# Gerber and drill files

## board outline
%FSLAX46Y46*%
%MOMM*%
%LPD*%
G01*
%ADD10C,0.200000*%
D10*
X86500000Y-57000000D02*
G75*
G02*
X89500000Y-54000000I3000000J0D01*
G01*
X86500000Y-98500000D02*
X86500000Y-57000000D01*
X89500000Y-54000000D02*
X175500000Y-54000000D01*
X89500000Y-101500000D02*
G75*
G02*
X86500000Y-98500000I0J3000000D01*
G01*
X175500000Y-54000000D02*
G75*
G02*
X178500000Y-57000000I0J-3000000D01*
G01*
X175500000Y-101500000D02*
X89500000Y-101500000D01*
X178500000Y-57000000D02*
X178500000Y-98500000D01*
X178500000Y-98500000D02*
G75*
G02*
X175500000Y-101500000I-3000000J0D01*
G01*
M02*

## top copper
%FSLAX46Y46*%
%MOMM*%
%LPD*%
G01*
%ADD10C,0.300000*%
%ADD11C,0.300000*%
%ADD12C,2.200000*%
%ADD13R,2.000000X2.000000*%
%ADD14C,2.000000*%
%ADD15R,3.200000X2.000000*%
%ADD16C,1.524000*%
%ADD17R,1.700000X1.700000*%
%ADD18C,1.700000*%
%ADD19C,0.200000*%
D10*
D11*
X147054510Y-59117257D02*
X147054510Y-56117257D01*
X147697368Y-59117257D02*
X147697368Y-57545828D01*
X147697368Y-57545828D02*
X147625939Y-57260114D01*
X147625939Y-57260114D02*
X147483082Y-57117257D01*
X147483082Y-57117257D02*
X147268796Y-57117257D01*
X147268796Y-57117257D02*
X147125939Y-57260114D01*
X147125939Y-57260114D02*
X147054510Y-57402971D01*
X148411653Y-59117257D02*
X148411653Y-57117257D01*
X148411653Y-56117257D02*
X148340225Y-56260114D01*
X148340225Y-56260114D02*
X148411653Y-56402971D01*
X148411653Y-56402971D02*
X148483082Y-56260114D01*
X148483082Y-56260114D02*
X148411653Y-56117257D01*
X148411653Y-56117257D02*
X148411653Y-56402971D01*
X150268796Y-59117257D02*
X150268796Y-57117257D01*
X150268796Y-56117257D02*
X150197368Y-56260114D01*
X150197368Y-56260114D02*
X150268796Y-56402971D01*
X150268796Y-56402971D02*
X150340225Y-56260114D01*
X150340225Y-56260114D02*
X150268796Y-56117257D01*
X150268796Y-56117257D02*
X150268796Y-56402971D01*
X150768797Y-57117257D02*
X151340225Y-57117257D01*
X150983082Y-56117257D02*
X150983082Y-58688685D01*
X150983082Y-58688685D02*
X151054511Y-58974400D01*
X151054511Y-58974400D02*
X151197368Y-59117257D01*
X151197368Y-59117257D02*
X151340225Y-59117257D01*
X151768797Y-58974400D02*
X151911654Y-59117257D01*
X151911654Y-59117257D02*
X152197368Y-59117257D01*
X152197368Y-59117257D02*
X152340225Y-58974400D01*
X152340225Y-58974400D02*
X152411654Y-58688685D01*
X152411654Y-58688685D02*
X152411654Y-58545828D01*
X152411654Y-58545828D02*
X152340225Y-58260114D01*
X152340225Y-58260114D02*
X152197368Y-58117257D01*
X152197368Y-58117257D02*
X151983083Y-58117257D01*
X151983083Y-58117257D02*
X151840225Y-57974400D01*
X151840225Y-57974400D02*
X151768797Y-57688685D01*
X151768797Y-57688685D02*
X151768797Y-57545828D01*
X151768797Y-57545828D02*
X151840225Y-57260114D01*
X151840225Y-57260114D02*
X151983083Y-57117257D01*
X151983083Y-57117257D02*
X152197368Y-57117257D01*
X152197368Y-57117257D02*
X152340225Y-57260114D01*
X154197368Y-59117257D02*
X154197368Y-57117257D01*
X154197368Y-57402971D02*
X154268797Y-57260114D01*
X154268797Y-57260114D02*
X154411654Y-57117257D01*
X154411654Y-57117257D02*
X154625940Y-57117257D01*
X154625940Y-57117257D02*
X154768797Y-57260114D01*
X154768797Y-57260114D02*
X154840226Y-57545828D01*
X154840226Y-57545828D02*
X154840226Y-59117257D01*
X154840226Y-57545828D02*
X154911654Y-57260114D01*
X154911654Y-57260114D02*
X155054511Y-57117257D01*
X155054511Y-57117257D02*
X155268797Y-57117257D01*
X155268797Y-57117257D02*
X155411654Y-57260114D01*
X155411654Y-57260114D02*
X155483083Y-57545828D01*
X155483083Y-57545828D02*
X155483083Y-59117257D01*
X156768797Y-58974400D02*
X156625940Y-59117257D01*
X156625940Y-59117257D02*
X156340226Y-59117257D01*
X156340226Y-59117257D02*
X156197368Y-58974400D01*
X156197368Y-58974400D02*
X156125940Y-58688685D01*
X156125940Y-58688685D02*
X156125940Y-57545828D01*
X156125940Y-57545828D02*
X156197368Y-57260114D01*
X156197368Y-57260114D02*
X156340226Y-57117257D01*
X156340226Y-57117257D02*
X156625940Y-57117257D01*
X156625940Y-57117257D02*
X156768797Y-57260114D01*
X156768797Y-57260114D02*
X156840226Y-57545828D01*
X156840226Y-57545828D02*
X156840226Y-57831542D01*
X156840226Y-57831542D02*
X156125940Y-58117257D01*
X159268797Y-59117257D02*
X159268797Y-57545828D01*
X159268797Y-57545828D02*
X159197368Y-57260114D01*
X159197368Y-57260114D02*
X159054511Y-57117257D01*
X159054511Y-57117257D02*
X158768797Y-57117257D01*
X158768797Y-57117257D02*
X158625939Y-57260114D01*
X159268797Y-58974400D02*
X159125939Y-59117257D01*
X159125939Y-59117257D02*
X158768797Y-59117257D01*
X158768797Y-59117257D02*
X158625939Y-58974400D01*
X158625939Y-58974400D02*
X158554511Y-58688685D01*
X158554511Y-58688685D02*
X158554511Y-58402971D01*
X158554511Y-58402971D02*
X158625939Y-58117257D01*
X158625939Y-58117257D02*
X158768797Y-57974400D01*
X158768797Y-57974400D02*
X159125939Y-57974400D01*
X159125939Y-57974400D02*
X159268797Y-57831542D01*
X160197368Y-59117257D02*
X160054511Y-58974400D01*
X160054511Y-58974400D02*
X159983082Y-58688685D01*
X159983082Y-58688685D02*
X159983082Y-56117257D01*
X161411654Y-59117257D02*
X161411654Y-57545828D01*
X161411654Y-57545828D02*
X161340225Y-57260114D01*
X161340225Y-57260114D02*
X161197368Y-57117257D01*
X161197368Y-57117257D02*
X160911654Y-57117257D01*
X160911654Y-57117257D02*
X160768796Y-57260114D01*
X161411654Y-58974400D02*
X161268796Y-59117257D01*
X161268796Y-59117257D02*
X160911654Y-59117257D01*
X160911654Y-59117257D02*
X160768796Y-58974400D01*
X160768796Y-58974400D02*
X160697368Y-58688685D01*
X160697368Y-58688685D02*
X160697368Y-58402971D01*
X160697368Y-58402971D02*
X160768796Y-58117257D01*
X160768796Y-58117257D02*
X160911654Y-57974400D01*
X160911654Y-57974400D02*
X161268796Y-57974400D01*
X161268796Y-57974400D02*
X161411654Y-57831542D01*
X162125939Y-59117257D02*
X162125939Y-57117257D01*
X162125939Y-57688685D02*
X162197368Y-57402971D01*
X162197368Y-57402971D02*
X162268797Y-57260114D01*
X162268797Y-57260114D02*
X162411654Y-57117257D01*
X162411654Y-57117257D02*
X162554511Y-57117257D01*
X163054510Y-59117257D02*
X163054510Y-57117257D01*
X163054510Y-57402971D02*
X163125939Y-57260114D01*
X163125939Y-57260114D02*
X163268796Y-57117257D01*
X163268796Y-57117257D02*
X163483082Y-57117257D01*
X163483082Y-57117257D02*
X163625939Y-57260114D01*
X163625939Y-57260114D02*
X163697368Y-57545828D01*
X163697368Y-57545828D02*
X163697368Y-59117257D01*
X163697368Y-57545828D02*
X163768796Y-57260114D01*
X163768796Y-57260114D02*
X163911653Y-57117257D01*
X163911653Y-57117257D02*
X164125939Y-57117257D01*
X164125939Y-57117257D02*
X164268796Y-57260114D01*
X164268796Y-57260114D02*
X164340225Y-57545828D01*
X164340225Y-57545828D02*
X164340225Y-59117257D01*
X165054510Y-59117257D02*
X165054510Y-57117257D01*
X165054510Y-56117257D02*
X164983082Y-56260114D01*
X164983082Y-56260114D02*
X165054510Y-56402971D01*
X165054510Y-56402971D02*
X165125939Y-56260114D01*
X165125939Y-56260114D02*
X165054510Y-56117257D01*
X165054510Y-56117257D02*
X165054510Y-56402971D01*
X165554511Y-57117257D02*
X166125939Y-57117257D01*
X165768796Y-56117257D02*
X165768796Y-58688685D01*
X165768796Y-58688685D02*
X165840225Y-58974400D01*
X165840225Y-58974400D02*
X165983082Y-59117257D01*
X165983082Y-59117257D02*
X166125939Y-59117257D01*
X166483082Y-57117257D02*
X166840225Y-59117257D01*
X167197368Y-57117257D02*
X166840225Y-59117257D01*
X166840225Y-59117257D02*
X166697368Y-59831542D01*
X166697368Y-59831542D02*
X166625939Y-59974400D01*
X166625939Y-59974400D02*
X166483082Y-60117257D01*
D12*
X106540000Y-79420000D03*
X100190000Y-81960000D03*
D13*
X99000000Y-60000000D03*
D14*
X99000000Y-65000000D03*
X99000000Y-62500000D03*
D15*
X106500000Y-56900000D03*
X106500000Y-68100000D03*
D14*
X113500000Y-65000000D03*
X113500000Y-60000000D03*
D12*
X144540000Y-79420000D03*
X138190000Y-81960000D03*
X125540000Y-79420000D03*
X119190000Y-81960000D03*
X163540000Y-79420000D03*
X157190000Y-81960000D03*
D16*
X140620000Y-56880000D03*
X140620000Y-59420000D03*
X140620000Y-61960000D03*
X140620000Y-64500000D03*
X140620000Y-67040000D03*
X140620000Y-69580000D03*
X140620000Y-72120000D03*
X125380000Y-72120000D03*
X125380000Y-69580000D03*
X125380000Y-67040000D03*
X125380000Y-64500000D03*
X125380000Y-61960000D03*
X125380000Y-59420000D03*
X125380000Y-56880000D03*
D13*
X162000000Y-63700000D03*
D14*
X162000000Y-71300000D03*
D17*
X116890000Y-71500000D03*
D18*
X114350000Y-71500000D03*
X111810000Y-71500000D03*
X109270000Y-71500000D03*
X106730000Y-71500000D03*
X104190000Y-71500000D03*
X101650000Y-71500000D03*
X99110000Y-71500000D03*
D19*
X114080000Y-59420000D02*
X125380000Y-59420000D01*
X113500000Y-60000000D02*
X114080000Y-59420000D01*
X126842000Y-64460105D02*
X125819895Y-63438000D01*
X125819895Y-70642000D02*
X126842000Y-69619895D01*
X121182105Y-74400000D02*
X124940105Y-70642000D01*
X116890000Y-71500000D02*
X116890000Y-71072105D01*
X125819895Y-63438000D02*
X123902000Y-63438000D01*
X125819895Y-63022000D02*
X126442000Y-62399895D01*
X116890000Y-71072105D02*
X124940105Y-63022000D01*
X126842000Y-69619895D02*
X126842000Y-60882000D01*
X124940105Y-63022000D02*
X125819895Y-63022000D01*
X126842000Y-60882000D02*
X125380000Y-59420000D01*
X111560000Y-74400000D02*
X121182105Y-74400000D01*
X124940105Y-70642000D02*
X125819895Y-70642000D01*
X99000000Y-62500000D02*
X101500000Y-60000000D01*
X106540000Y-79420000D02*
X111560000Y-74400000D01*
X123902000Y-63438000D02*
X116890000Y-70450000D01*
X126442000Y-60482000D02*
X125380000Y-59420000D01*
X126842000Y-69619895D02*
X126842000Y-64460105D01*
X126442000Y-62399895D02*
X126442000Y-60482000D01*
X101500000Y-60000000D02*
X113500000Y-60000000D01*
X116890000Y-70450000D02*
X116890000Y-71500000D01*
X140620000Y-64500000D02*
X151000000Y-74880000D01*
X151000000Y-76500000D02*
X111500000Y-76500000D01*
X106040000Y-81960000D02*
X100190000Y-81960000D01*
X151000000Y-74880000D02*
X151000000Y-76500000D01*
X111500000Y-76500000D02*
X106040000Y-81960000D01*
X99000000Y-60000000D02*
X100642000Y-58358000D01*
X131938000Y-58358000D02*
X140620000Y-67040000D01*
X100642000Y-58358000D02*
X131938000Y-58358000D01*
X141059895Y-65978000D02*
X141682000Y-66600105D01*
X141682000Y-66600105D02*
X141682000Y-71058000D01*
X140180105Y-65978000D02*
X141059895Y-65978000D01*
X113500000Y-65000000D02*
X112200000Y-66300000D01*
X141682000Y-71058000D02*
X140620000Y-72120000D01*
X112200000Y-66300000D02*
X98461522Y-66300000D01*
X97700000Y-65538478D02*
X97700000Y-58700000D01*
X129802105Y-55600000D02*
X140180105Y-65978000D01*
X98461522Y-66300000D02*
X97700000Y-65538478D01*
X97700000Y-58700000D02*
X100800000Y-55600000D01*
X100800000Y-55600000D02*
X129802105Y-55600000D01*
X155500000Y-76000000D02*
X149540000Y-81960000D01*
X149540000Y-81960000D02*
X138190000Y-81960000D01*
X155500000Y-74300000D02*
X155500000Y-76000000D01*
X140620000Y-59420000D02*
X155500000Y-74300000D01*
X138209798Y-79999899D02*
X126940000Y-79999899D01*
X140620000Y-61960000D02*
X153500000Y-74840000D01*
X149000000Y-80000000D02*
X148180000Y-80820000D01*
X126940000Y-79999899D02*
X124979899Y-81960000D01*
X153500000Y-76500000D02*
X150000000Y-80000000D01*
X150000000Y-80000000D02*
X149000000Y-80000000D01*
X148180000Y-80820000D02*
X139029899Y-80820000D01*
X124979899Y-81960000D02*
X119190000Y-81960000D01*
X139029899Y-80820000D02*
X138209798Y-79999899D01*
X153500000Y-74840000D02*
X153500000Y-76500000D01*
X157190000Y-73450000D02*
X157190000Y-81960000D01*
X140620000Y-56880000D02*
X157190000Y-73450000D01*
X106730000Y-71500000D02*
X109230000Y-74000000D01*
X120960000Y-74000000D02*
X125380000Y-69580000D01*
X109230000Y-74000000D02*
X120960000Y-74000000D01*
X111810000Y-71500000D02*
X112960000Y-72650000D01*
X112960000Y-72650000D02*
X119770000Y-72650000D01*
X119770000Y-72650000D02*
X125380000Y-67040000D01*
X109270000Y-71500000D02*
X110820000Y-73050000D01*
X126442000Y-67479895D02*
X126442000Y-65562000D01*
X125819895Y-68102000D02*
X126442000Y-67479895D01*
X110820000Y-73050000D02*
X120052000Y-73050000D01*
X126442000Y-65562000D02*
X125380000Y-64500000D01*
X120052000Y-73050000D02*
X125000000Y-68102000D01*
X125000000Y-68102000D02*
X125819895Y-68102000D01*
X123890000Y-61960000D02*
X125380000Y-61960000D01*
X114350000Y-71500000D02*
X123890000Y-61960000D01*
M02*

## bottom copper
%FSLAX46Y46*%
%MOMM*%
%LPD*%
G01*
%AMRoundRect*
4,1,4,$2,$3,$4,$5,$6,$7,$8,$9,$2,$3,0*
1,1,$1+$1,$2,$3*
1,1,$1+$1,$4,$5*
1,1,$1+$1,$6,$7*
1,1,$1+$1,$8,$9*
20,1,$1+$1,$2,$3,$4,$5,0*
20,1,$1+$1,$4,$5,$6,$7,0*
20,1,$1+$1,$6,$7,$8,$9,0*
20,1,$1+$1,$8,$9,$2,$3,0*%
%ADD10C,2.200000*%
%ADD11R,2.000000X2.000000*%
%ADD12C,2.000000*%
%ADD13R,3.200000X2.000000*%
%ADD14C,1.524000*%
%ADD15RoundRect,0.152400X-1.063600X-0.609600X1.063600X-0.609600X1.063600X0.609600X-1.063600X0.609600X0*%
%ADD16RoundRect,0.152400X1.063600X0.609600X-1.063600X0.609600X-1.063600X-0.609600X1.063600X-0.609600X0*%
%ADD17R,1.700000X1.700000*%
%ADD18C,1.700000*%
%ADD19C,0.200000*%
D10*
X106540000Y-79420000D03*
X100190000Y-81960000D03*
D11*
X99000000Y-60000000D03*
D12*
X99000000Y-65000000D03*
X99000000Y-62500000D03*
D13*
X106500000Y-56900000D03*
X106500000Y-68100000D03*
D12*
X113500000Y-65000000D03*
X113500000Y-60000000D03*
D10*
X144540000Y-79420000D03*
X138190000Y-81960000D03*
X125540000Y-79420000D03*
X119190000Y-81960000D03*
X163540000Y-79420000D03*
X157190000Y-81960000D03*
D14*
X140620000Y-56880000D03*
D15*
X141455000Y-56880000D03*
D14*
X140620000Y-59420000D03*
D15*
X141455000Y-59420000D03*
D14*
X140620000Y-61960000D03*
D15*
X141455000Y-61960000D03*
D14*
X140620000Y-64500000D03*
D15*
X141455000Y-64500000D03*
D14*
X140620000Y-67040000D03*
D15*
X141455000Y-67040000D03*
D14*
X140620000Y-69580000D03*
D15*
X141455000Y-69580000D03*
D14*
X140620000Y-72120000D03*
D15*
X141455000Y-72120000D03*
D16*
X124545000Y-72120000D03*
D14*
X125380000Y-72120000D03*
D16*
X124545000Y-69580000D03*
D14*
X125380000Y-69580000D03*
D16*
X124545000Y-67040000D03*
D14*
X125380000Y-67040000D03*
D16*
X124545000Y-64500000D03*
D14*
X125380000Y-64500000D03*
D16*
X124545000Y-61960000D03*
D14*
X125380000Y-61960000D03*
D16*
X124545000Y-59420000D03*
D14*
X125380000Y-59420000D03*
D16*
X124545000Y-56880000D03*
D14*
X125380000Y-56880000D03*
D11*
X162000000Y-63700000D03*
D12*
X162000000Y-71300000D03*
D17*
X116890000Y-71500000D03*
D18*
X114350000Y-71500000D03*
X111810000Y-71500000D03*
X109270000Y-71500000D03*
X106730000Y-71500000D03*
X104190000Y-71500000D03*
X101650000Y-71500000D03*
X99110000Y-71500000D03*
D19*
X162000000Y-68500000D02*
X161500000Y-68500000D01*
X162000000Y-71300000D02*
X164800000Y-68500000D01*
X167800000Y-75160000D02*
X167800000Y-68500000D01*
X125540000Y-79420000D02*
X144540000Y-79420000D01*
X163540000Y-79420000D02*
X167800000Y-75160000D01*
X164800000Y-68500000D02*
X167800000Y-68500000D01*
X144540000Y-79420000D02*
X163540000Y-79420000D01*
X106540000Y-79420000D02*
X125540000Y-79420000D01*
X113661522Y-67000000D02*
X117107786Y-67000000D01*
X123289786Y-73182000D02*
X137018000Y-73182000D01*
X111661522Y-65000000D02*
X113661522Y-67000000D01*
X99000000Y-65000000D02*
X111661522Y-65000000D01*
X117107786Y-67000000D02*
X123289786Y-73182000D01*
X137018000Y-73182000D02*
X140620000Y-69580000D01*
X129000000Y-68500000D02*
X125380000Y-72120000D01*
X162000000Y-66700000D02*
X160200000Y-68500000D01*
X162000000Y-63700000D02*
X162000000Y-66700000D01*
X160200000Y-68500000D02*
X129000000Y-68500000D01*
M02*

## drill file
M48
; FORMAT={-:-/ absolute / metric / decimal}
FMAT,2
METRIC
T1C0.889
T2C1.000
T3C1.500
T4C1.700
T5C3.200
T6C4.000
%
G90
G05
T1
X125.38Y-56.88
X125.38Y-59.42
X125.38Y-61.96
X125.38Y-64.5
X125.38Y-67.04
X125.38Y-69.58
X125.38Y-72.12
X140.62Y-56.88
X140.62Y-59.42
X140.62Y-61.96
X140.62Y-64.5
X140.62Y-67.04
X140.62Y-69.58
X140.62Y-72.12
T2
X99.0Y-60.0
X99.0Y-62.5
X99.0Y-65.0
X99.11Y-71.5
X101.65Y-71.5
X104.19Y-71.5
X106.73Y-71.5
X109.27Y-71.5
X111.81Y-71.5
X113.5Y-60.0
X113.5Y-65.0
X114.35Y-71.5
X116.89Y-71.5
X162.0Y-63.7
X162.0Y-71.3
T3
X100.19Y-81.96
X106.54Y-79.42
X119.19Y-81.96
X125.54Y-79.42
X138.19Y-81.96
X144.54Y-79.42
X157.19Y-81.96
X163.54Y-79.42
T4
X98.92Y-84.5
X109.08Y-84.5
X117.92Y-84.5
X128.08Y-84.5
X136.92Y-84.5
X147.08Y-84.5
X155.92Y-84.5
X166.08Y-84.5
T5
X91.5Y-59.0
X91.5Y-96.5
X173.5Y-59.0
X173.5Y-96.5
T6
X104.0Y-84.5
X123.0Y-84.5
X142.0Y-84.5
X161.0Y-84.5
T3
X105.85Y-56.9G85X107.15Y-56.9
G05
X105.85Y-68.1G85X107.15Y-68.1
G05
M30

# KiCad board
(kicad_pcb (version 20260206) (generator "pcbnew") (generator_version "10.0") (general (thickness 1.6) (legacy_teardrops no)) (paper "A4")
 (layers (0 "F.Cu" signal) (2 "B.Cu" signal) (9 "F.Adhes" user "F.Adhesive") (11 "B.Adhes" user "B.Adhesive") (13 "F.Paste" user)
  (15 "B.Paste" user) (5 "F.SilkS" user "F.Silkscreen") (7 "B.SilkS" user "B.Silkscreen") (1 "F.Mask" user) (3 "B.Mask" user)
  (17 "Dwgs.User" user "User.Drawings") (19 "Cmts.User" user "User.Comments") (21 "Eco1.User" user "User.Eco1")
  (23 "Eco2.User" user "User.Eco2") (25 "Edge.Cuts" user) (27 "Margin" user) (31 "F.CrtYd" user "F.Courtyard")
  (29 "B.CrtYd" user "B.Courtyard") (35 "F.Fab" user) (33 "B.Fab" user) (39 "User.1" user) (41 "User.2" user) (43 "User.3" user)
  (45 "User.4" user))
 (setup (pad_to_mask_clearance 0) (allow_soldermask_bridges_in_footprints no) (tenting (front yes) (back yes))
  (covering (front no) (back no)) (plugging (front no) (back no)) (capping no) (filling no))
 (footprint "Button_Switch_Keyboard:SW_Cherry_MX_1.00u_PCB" (layer "F.Cu") (at 106.54 79.42)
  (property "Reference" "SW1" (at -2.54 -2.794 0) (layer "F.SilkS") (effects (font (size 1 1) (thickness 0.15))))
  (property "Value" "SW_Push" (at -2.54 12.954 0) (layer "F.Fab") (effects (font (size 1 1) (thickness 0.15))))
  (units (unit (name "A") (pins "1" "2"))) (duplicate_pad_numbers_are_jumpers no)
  (pad "" np_thru_hole circle (at -7.62 5.08) (size 1.7 1.7) (drill 1.7) (layers "*.Cu" "*.Mask"))
  (pad "" np_thru_hole circle (at -2.54 5.08) (size 4 4) (drill 4) (layers "*.Cu" "*.Mask"))
  (pad "" np_thru_hole circle (at 2.54 5.08) (size 1.7 1.7) (drill 1.7) (layers "*.Cu" "*.Mask"))
  (pad "1" thru_hole circle (at 0 0) (size 2.2 2.2) (drill 1.5) (layers "*.Cu" "*.Mask") (remove_unused_layers no) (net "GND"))
  (pad "2" thru_hole circle (at -6.35 2.54) (size 2.2 2.2) (drill 1.5) (layers "*.Cu" "*.Mask") (remove_unused_layers no)
   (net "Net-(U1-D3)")))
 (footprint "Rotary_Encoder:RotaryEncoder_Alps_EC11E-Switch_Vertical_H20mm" (layer "F.Cu") (at 99 60)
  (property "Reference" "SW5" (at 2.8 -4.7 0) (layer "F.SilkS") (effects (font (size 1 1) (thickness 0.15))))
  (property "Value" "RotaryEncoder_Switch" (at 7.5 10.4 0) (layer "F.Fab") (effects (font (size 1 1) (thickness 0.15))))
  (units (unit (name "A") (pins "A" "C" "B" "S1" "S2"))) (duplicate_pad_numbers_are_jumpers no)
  (pad "A" thru_hole rect (at 0 0) (size 2 2) (drill 1) (layers "*.Cu" "*.Mask") (remove_unused_layers no) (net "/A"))
  (pad "B" thru_hole circle (at 0 5) (size 2 2) (drill 1) (layers "*.Cu" "*.Mask") (remove_unused_layers no) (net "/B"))
  (pad "C" thru_hole circle (at 0 2.5) (size 2 2) (drill 1) (layers "*.Cu" "*.Mask") (remove_unused_layers no) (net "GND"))
  (pad "MP" thru_hole rect (at 7.5 -3.1) (size 3.2 2) (drill oval 2.8 1.5) (layers "*.Cu" "*.Mask") (remove_unused_layers no))
  (pad "MP" thru_hole rect (at 7.5 8.1) (size 3.2 2) (drill oval 2.8 1.5) (layers "*.Cu" "*.Mask") (remove_unused_layers no))
  (pad "S1" thru_hole circle (at 14.5 5) (size 2 2) (drill 1) (layers "*.Cu" "*.Mask") (remove_unused_layers no) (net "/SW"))
  (pad "S2" thru_hole circle (at 14.5 0) (size 2 2) (drill 1) (layers "*.Cu" "*.Mask") (remove_unused_layers no) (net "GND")))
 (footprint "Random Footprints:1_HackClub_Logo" (layer "F.Cu") (at 155.5 68.5)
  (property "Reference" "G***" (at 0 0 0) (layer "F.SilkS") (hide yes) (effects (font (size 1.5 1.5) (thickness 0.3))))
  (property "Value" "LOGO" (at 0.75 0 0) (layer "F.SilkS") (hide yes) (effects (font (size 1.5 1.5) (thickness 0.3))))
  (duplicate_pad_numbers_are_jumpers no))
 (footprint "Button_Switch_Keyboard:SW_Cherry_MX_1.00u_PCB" (layer "F.Cu") (at 144.54 79.42)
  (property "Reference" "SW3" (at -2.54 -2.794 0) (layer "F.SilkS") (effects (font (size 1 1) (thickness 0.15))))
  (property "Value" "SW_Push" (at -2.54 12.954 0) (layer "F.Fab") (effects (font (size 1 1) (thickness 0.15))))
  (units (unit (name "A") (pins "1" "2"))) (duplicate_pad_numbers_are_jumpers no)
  (pad "" np_thru_hole circle (at -7.62 5.08) (size 1.7 1.7) (drill 1.7) (layers "*.Cu" "*.Mask"))
  (pad "" np_thru_hole circle (at -2.54 5.08) (size 4 4) (drill 4) (layers "*.Cu" "*.Mask"))
  (pad "" np_thru_hole circle (at 2.54 5.08) (size 1.7 1.7) (drill 1.7) (layers "*.Cu" "*.Mask"))
  (pad "1" thru_hole circle (at 0 0) (size 2.2 2.2) (drill 1.5) (layers "*.Cu" "*.Mask") (remove_unused_layers no) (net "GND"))
  (pad "2" thru_hole circle (at -6.35 2.54) (size 2.2 2.2) (drill 1.5) (layers "*.Cu" "*.Mask") (remove_unused_layers no)
   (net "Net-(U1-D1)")))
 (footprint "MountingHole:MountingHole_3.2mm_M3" (layer "F.Cu") (at 91.5 96.5 180)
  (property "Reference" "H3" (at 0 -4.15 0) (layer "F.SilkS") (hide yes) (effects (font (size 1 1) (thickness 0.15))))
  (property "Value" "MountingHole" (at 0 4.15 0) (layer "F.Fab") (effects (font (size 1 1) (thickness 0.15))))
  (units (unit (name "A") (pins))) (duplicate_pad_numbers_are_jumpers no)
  (pad "" np_thru_hole circle (at 0 0 180) (size 3.2 3.2) (drill 3.2) (layers "*.Cu" "*.Mask")))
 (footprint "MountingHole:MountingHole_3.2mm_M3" (layer "F.Cu") (at 91.5 59)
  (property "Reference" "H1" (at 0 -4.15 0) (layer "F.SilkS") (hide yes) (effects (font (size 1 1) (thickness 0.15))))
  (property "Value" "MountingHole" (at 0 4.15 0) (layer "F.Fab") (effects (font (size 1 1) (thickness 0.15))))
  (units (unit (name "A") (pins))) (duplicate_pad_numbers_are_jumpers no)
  (pad "" np_thru_hole circle (at 0 0) (size 3.2 3.2) (drill 3.2) (layers "*.Cu" "*.Mask")))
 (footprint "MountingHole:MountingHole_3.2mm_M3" (layer "F.Cu") (at 173.5 59)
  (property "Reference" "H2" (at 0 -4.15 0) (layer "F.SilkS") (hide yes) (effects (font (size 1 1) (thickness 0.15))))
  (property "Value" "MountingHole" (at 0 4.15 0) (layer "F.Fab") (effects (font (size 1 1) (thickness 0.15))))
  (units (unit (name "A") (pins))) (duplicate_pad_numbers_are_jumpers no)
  (pad "" np_thru_hole circle (at 0 0) (size 3.2 3.2) (drill 3.2) (layers "*.Cu" "*.Mask")))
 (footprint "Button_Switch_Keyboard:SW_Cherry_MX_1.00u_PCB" (layer "F.Cu") (at 125.54 79.42)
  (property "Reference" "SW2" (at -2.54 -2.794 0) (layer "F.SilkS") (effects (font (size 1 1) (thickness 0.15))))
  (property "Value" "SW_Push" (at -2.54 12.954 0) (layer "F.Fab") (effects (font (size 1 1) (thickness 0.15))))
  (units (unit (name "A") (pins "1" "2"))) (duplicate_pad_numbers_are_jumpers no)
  (pad "" np_thru_hole circle (at -7.62 5.08) (size 1.7 1.7) (drill 1.7) (layers "*.Cu" "*.Mask"))
  (pad "" np_thru_hole circle (at -2.54 5.08) (size 4 4) (drill 4) (layers "*.Cu" "*.Mask"))
  (pad "" np_thru_hole circle (at 2.54 5.08) (size 1.7 1.7) (drill 1.7) (layers "*.Cu" "*.Mask"))
  (pad "1" thru_hole circle (at 0 0) (size 2.2 2.2) (drill 1.5) (layers "*.Cu" "*.Mask") (remove_unused_layers no) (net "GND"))
  (pad "2" thru_hole circle (at -6.35 2.54) (size 2.2 2.2) (drill 1.5) (layers "*.Cu" "*.Mask") (remove_unused_layers no)
   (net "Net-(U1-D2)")))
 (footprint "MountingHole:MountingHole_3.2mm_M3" (layer "F.Cu") (at 173.5 96.5 180)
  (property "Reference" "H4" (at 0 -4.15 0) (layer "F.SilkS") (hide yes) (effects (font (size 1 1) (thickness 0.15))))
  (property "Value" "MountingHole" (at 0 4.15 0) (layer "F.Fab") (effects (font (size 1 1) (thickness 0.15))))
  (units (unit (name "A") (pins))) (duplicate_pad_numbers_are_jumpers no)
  (pad "" np_thru_hole circle (at 0 0 180) (size 3.2 3.2) (drill 3.2) (layers "*.Cu" "*.Mask")))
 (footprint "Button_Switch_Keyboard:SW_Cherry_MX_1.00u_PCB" (layer "F.Cu") (at 163.54 79.42)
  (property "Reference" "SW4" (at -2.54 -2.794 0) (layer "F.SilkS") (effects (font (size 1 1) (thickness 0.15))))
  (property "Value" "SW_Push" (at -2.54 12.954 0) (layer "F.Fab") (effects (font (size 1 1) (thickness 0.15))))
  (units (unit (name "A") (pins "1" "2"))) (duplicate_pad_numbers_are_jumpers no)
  (pad "" np_thru_hole circle (at -7.62 5.08) (size 1.7 1.7) (drill 1.7) (layers "*.Cu" "*.Mask"))
  (pad "" np_thru_hole circle (at -2.54 5.08) (size 4 4) (drill 4) (layers "*.Cu" "*.Mask"))
  (pad "" np_thru_hole circle (at 2.54 5.08) (size 1.7 1.7) (drill 1.7) (layers "*.Cu" "*.Mask"))
  (pad "1" thru_hole circle (at 0 0) (size 2.2 2.2) (drill 1.5) (layers "*.Cu" "*.Mask") (remove_unused_layers no) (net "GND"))
  (pad "2" thru_hole circle (at -6.35 2.54) (size 2.2 2.2) (drill 1.5) (layers "*.Cu" "*.Mask") (remove_unused_layers no)
   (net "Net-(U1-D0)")))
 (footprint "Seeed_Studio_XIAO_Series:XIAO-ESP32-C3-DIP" (layer "B.Cu") (at 133 64.5 90)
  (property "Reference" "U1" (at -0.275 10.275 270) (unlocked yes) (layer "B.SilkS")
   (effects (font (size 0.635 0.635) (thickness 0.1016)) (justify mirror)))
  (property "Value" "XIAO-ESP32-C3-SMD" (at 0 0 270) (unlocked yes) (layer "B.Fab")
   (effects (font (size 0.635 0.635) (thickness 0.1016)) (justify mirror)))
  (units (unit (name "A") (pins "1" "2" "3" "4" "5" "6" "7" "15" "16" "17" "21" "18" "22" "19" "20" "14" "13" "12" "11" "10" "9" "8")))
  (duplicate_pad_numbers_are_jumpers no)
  (pad "1" thru_hole circle (at 7.62 7.62) (size 1.524 1.524) (drill 0.889) (layers "*.Cu" "*.Mask") (remove_unused_layers no)
   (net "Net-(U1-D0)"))
  (pad "1" smd roundrect (at 7.62 8.455) (size 2.432 1.524) (layers "B.Cu" "B.Mask") (roundrect_rratio 0.1) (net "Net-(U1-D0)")
   (thermal_bridge_angle 45))
  (pad "2" thru_hole circle (at 5.08 7.62) (size 1.524 1.524) (drill 0.889) (layers "*.Cu" "*.Mask") (remove_unused_layers no)
   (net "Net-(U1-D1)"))
  (pad "2" smd roundrect (at 5.08 8.455) (size 2.432 1.524) (layers "B.Cu" "B.Mask") (roundrect_rratio 0.1) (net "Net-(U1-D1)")
   (thermal_bridge_angle 45))
  (pad "3" thru_hole circle (at 2.54 7.62) (size 1.524 1.524) (drill 0.889) (layers "*.Cu" "*.Mask") (remove_unused_layers no)
   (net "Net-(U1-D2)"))
  (pad "3" smd roundrect (at 2.54 8.455) (size 2.432 1.524) (layers "B.Cu" "B.Mask") (roundrect_rratio 0.1) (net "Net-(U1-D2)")
   (thermal_bridge_angle 45))
  (pad "4" thru_hole circle (at 0 7.62) (size 1.524 1.524) (drill 0.889) (layers "*.Cu" "*.Mask") (remove_unused_layers no)
   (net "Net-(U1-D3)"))
  (pad "4" smd roundrect (at 0 8.455) (size 2.432 1.524) (layers "B.Cu" "B.Mask") (roundrect_rratio 0.1) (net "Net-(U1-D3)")
   (thermal_bridge_angle 45))
  (pad "5" thru_hole circle (at -2.54 7.62) (size 1.524 1.524) (drill 0.889) (layers "*.Cu" "*.Mask") (remove_unused_layers no) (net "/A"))
  (pad "5" smd roundrect (at -2.54 8.455) (size 2.432 1.524) (layers "B.Cu" "B.Mask") (roundrect_rratio 0.1) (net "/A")
   (thermal_bridge_angle 45))
  (pad "6" thru_hole circle (at -5.08 7.62) (size 1.524 1.524) (drill 0.889) (layers "*.Cu" "*.Mask") (remove_unused_layers no) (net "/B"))
  (pad "6" smd roundrect (at -5.08 8.455) (size 2.432 1.524) (layers "B.Cu" "B.Mask") (roundrect_rratio 0.1) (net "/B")
   (thermal_bridge_angle 45))
  (pad "7" thru_hole circle (at -7.62 7.62) (size 1.524 1.524) (drill 0.889) (layers "*.Cu" "*.Mask") (remove_unused_layers no) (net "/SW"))
  (pad "7" smd roundrect (at -7.62 8.455) (size 2.432 1.524) (layers "B.Cu" "B.Mask") (roundrect_rratio 0.1) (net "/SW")
   (thermal_bridge_angle 45))
  (pad "8" smd roundrect (at -7.62 -8.455 180) (size 2.432 1.524) (layers "B.Cu" "B.Mask") (roundrect_rratio 0.1) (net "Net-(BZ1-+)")
   (thermal_bridge_angle 45))
  (pad "8" thru_hole circle (at -7.62 -7.62 180) (size 1.524 1.524) (drill 0.889) (layers "*.Cu" "*.Mask") (remove_unused_layers no)
   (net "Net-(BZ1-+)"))
  (pad "9" smd roundrect (at -5.08 -8.455 180) (size 2.432 1.524) (layers "B.Cu" "B.Mask") (roundrect_rratio 0.1) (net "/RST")
   (thermal_bridge_angle 45))
  (pad "9" thru_hole circle (at -5.08 -7.62 180) (size 1.524 1.524) (drill 0.889) (layers "*.Cu" "*.Mask") (remove_unused_layers no)
   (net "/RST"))
  (pad "10" smd roundrect (at -2.54 -8.455 180) (size 2.432 1.524) (layers "B.Cu" "B.Mask") (roundrect_rratio 0.1) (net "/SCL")
   (thermal_bridge_angle 45))
  (pad "10" thru_hole circle (at -2.54 -7.62 180) (size 1.524 1.524) (drill 0.889) (layers "*.Cu" "*.Mask") (remove_unused_layers no)
   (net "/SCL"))
  (pad "11" smd roundrect (at 0 -8.455 180) (size 2.432 1.524) (layers "B.Cu" "B.Mask") (roundrect_rratio 0.1) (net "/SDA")
   (thermal_bridge_angle 45))
  (pad "11" thru_hole circle (at 0 -7.62 180) (size 1.524 1.524) (drill 0.889) (layers "*.Cu" "*.Mask") (remove_unused_layers no)
   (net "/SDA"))
  (pad "12" smd roundrect (at 2.54 -8.455 180) (size 2.432 1.524) (layers "B.Cu" "B.Mask") (roundrect_rratio 0.1) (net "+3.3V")
   (thermal_bridge_angle 45))
  (pad "12" thru_hole circle (at 2.54 -7.62 180) (size 1.524 1.524) (drill 0.889) (layers "*.Cu" "*.Mask") (remove_unused_layers no)
   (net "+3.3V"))
  (pad "13" smd roundrect (at 5.08 -8.455 180) (size 2.432 1.524) (layers "B.Cu" "B.Mask") (roundrect_rratio 0.1) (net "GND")
   (thermal_bridge_angle 45))
  (pad "13" thru_hole circle (at 5.08 -7.62 180) (size 1.524 1.524) (drill 0.889) (layers "*.Cu" "*.Mask") (remove_unused_layers no)
   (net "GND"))
  (pad "14" smd roundrect (at 7.62 -8.455 180) (size 2.432 1.524) (layers "B.Cu" "B.Mask") (roundrect_rratio 0.1)
   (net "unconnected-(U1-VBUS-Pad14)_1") (thermal_bridge_angle 45))
  (pad "14" thru_hole circle (at 7.62 -7.62 180) (size 1.524 1.524) (drill 0.889) (layers "*.Cu" "*.Mask") (remove_unused_layers no)
   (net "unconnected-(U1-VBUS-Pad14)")))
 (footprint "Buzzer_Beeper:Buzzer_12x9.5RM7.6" (layer "B.Cu") (at 162 63.7 -90)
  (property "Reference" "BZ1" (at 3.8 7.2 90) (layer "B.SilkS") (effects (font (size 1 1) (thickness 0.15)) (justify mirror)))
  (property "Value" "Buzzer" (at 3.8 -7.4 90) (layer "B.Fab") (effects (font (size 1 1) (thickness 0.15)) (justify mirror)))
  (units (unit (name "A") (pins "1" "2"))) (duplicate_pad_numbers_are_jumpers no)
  (pad "1" thru_hole rect (at 0 0 270) (size 2 2) (drill 1) (layers "*.Cu" "*.Mask") (remove_unused_layers no) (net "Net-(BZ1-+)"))
  (pad "2" thru_hole circle (at 7.6 0 270) (size 2 2) (drill 1) (layers "*.Cu" "*.Mask") (remove_unused_layers no) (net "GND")))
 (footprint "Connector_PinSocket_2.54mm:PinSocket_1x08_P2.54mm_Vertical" (layer "B.Cu") (at 116.89 71.5 90)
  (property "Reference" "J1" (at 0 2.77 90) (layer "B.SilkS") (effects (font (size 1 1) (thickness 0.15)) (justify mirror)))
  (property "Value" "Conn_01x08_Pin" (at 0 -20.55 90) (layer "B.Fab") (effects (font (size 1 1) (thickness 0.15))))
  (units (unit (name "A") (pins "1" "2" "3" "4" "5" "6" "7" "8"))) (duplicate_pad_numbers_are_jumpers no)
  (pad "1" thru_hole rect (at 0 0 90) (size 1.7 1.7) (drill 1) (layers "*.Cu" "*.Mask") (remove_unused_layers no) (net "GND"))
  (pad "2" thru_hole circle (at 0 -2.54 90) (size 1.7 1.7) (drill 1) (layers "*.Cu" "*.Mask") (remove_unused_layers no) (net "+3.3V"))
  (pad "3" thru_hole circle (at 0 -5.08 90) (size 1.7 1.7) (drill 1) (layers "*.Cu" "*.Mask") (remove_unused_layers no) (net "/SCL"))
  (pad "4" thru_hole circle (at 0 -7.62 90) (size 1.7 1.7) (drill 1) (layers "*.Cu" "*.Mask") (remove_unused_layers no) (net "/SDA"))
  (pad "5" thru_hole circle (at 0 -10.16 90) (size 1.7 1.7) (drill 1) (layers "*.Cu" "*.Mask") (remove_unused_layers no) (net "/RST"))
  (pad "6" thru_hole circle (at 0 -12.7 90) (size 1.7 1.7) (drill 1) (layers "*.Cu" "*.Mask") (remove_unused_layers no) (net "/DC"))
  (pad "7" thru_hole circle (at 0 -15.24 90) (size 1.7 1.7) (drill 1) (layers "*.Cu" "*.Mask") (remove_unused_layers no) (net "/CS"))
  (pad "8" thru_hole circle (at 0 -17.78 90) (size 1.7 1.7) (drill 1) (layers "*.Cu" "*.Mask") (remove_unused_layers no) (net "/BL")))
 (gr_arc (start 86.5 57) (mid 87.37868 54.87868) (end 89.5 54) (stroke (width 0.2) (type default)) (layer "Edge.Cuts"))
 (gr_line (start 86.5 98.5) (end 86.5 57) (stroke (width 0.2) (type default)) (layer "Edge.Cuts"))
 (gr_line (start 89.5 54) (end 175.5 54) (stroke (width 0.2) (type default)) (layer "Edge.Cuts"))
 (gr_arc (start 89.5 101.5) (mid 87.37868 100.62132) (end 86.5 98.5) (stroke (width 0.2) (type default)) (layer "Edge.Cuts"))
 (gr_arc (start 175.5 54) (mid 177.62132 54.87868) (end 178.5 57) (stroke (width 0.2) (type default)) (layer "Edge.Cuts"))
 (gr_line (start 175.5 101.5) (end 89.5 101.5) (stroke (width 0.2) (type default)) (layer "Edge.Cuts"))
 (gr_line (start 178.5 57) (end 178.5 98.5) (stroke (width 0.2) (type default)) (layer "Edge.Cuts"))
 (gr_arc (start 178.5 98.5) (mid 177.62132 100.62132) (end 175.5 101.5) (stroke (width 0.2) (type default)) (layer "Edge.Cuts"))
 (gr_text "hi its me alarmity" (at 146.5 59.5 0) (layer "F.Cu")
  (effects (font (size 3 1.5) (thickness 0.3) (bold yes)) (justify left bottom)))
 (segment (start 162 68.5) (end 161.5 68.5) (width 0.2) (layer "B.Cu") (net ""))
 (segment (start 114.08 59.42) (end 125.38 59.42) (width 0.2) (layer "F.Cu") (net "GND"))
 (segment (start 113.5 60) (end 114.08 59.42) (width 0.2) (layer "F.Cu") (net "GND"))
 (segment (start 126.842 64.460105) (end 125.819895 63.438) (width 0.2) (layer "F.Cu") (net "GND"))
 (segment (start 125.819895 70.642) (end 126.842 69.619895) (width 0.2) (layer "F.Cu") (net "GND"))
 (segment (start 121.182105 74.4) (end 124.940105 70.642) (width 0.2) (layer "F.Cu") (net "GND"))
 (segment (start 116.89 71.5) (end 116.89 71.072105) (width 0.2) (layer "F.Cu") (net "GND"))
 (segment (start 125.819895 63.438) (end 123.902 63.438) (width 0.2) (layer "F.Cu") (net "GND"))
 (segment (start 125.819895 63.022) (end 126.442 62.399895) (width 0.2) (layer "F.Cu") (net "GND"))
 (segment (start 116.89 71.072105) (end 124.940105 63.022) (width 0.2) (layer "F.Cu") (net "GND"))
 (segment (start 126.842 69.619895) (end 126.842 60.882) (width 0.2) (layer "F.Cu") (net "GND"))
 (segment (start 124.940105 63.022) (end 125.819895 63.022) (width 0.2) (layer "F.Cu") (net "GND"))
 (segment (start 126.842 60.882) (end 125.38 59.42) (width 0.2) (layer "F.Cu") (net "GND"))
 (segment (start 111.56 74.4) (end 121.182105 74.4) (width 0.2) (layer "F.Cu") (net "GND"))
 (segment (start 124.940105 70.642) (end 125.819895 70.642) (width 0.2) (layer "F.Cu") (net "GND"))
 (segment (start 99 62.5) (end 101.5 60) (width 0.2) (layer "F.Cu") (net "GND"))
 (segment (start 106.54 79.42) (end 111.56 74.4) (width 0.2) (layer "F.Cu") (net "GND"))
 (segment (start 123.902 63.438) (end 116.89 70.45) (width 0.2) (layer "F.Cu") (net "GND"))
 (segment (start 126.442 60.482) (end 125.38 59.42) (width 0.2) (layer "F.Cu") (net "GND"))
 (segment (start 126.842 69.619895) (end 126.842 64.460105) (width 0.2) (layer "F.Cu") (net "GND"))
 (segment (start 126.442 62.399895) (end 126.442 60.482) (width 0.2) (layer "F.Cu") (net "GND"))
 (segment (start 101.5 60) (end 113.5 60) (width 0.2) (layer "F.Cu") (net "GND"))
 (segment (start 116.89 70.45) (end 116.89 71.5) (width 0.2) (layer "F.Cu") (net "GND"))
 (segment (start 162 71.3) (end 164.8 68.5) (width 0.2) (layer "B.Cu") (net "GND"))
 (segment (start 167.8 75.16) (end 167.8 68.5) (width 0.2) (layer "B.Cu") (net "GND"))
 (segment (start 125.54 79.42) (end 144.54 79.42) (width 0.2) (layer "B.Cu") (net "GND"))
 (segment (start 163.54 79.42) (end 167.8 75.16) (width 0.2) (layer "B.Cu") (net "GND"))
 (segment (start 164.8 68.5) (end 167.8 68.5) (width 0.2) (layer "B.Cu") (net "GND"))
 (segment (start 144.54 79.42) (end 163.54 79.42) (width 0.2) (layer "B.Cu") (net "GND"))
 (segment (start 106.54 79.42) (end 125.54 79.42) (width 0.2) (layer "B.Cu") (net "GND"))
 (segment (start 140.62 64.5) (end 151 74.88) (width 0.2) (layer "F.Cu") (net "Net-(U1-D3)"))
 (segment (start 151 76.5) (end 111.5 76.5) (width 0.2) (layer "F.Cu") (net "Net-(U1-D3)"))
 (segment (start 106.04 81.96) (end 100.19 81.96) (width 0.2) (layer "F.Cu") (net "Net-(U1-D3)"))
 (segment (start 151 74.88) (end 151 76.5) (width 0.2) (layer "F.Cu") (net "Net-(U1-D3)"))
 (segment (start 111.5 76.5) (end 106.04 81.96) (width 0.2) (layer "F.Cu") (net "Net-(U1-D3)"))
 (segment (start 99 60) (end 100.642 58.358) (width 0.2) (layer "F.Cu") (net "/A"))
 (segment (start 131.938 58.358) (end 140.62 67.04) (width 0.2) (layer "F.Cu") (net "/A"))
 (segment (start 100.642 58.358) (end 131.938 58.358) (width 0.2) (layer "F.Cu") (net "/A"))
 (segment (start 113.661522 67) (end 117.107786 67) (width 0.2) (layer "B.Cu") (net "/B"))
 (segment (start 123.289786 73.182) (end 137.018 73.182) (width 0.2) (layer "B.Cu") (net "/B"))
 (segment (start 111.661522 65) (end 113.661522 67) (width 0.2) (layer "B.Cu") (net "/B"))
 (segment (start 99 65) (end 111.661522 65) (width 0.2) (layer "B.Cu") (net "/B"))
 (segment (start 117.107786 67) (end 123.289786 73.182) (width 0.2) (layer "B.Cu") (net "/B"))
 (segment (start 137.018 73.182) (end 140.62 69.58) (width 0.2) (layer "B.Cu") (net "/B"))
 (segment (start 141.059895 65.978) (end 141.682 66.600105) (width 0.2) (layer "F.Cu") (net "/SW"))
 (segment (start 141.682 66.600105) (end 141.682 71.058) (width 0.2) (layer "F.Cu") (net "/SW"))
 (segment (start 140.180105 65.978) (end 141.059895 65.978) (width 0.2) (layer "F.Cu") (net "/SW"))
 (segment (start 113.5 65) (end 112.2 66.3) (width 0.2) (layer "F.Cu") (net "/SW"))
 (segment (start 141.682 71.058) (end 140.62 72.12) (width 0.2) (layer "F.Cu") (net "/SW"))
 (segment (start 112.2 66.3) (end 98.461522 66.3) (width 0.2) (layer "F.Cu") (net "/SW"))
 (segment (start 97.7 65.538478) (end 97.7 58.7) (width 0.2) (layer "F.Cu") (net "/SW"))
 (segment (start 129.802105 55.6) (end 140.180105 65.978) (width 0.2) (layer "F.Cu") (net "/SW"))
 (segment (start 98.461522 66.3) (end 97.7 65.538478) (width 0.2) (layer "F.Cu") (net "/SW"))
 (segment (start 97.7 58.7) (end 100.8 55.6) (width 0.2) (layer "F.Cu") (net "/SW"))
 (segment (start 100.8 55.6) (end 129.802105 55.6) (width 0.2) (layer "F.Cu") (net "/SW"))
 (segment (start 155.5 76) (end 149.54 81.96) (width 0.2) (layer "F.Cu") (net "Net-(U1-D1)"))
 (segment (start 149.54 81.96) (end 138.19 81.96) (width 0.2) (layer "F.Cu") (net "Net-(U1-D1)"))
 (segment (start 155.5 74.3) (end 155.5 76) (width 0.2) (layer "F.Cu") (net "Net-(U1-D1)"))
 (segment (start 140.62 59.42) (end 155.5 74.3) (width 0.2) (layer "F.Cu") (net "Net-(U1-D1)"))
 (segment (start 138.209798 79.999899) (end 126.94 79.999899) (width 0.2) (layer "F.Cu") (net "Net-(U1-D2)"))
 (segment (start 140.62 61.96) (end 153.5 74.84) (width 0.2) (layer "F.Cu") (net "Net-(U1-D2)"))
 (segment (start 149 80) (end 148.18 80.82) (width 0.2) (layer "F.Cu") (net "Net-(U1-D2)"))
 (segment (start 126.94 79.999899) (end 124.979899 81.96) (width 0.2) (layer "F.Cu") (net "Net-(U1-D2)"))
 (segment (start 153.5 76.5) (end 150 80) (width 0.2) (layer "F.Cu") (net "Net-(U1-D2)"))
 (segment (start 150 80) (end 149 80) (width 0.2) (layer "F.Cu") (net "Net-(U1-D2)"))
 (segment (start 148.18 80.82) (end 139.029899 80.82) (width 0.2) (layer "F.Cu") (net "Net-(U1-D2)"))
 (segment (start 124.979899 81.96) (end 119.19 81.96) (width 0.2) (layer "F.Cu") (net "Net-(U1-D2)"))
 (segment (start 139.029899 80.82) (end 138.209798 79.999899) (width 0.2) (layer "F.Cu") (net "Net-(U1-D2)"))
 (segment (start 153.5 74.84) (end 153.5 76.5) (width 0.2) (layer "F.Cu") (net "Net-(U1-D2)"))
 (segment (start 157.19 73.45) (end 157.19 81.96) (width 0.2) (layer "F.Cu") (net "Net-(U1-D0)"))
 (segment (start 140.62 56.88) (end 157.19 73.45) (width 0.2) (layer "F.Cu") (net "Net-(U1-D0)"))
 (segment (start 129 68.5) (end 125.38 72.12) (width 0.2) (layer "B.Cu") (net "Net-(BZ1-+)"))
 (segment (start 162 66.7) (end 160.2 68.5) (width 0.2) (layer "B.Cu") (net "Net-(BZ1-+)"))
 (segment (start 162 63.7) (end 162 66.7) (width 0.2) (layer "B.Cu") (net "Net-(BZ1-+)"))
 (segment (start 160.2 68.5) (end 129 68.5) (width 0.2) (layer "B.Cu") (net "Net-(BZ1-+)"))
 (segment (start 106.73 71.5) (end 109.23 74) (width 0.2) (layer "F.Cu") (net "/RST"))
 (segment (start 120.96 74) (end 125.38 69.58) (width 0.2) (layer "F.Cu") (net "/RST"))
 (segment (start 109.23 74) (end 120.96 74) (width 0.2) (layer "F.Cu") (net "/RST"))
 (segment (start 111.81 71.5) (end 112.96 72.65) (width 0.2) (layer "F.Cu") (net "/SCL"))
 (segment (start 112.96 72.65) (end 119.77 72.65) (width 0.2) (layer "F.Cu") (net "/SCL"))
 (segment (start 119.77 72.65) (end 125.38 67.04) (width 0.2) (layer "F.Cu") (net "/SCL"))
 (segment (start 109.27 71.5) (end 110.82 73.05) (width 0.2) (layer "F.Cu") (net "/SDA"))
 (segment (start 126.442 67.479895) (end 126.442 65.562) (width 0.2) (layer "F.Cu") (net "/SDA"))
 (segment (start 125.819895 68.102) (end 126.442 67.479895) (width 0.2) (layer "F.Cu") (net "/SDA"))
 (segment (start 110.82 73.05) (end 120.052 73.05) (width 0.2) (layer "F.Cu") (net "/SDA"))
 (segment (start 126.442 65.562) (end 125.38 64.5) (width 0.2) (layer "F.Cu") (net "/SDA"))
 (segment (start 120.052 73.05) (end 125 68.102) (width 0.2) (layer "F.Cu") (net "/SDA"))
 (segment (start 125 68.102) (end 125.819895 68.102) (width 0.2) (layer "F.Cu") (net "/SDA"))
 (segment (start 123.89 61.96) (end 125.38 61.96) (width 0.2) (layer "F.Cu") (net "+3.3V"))
 (segment (start 114.35 71.5) (end 123.89 61.96) (width 0.2) (layer "F.Cu") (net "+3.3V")))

